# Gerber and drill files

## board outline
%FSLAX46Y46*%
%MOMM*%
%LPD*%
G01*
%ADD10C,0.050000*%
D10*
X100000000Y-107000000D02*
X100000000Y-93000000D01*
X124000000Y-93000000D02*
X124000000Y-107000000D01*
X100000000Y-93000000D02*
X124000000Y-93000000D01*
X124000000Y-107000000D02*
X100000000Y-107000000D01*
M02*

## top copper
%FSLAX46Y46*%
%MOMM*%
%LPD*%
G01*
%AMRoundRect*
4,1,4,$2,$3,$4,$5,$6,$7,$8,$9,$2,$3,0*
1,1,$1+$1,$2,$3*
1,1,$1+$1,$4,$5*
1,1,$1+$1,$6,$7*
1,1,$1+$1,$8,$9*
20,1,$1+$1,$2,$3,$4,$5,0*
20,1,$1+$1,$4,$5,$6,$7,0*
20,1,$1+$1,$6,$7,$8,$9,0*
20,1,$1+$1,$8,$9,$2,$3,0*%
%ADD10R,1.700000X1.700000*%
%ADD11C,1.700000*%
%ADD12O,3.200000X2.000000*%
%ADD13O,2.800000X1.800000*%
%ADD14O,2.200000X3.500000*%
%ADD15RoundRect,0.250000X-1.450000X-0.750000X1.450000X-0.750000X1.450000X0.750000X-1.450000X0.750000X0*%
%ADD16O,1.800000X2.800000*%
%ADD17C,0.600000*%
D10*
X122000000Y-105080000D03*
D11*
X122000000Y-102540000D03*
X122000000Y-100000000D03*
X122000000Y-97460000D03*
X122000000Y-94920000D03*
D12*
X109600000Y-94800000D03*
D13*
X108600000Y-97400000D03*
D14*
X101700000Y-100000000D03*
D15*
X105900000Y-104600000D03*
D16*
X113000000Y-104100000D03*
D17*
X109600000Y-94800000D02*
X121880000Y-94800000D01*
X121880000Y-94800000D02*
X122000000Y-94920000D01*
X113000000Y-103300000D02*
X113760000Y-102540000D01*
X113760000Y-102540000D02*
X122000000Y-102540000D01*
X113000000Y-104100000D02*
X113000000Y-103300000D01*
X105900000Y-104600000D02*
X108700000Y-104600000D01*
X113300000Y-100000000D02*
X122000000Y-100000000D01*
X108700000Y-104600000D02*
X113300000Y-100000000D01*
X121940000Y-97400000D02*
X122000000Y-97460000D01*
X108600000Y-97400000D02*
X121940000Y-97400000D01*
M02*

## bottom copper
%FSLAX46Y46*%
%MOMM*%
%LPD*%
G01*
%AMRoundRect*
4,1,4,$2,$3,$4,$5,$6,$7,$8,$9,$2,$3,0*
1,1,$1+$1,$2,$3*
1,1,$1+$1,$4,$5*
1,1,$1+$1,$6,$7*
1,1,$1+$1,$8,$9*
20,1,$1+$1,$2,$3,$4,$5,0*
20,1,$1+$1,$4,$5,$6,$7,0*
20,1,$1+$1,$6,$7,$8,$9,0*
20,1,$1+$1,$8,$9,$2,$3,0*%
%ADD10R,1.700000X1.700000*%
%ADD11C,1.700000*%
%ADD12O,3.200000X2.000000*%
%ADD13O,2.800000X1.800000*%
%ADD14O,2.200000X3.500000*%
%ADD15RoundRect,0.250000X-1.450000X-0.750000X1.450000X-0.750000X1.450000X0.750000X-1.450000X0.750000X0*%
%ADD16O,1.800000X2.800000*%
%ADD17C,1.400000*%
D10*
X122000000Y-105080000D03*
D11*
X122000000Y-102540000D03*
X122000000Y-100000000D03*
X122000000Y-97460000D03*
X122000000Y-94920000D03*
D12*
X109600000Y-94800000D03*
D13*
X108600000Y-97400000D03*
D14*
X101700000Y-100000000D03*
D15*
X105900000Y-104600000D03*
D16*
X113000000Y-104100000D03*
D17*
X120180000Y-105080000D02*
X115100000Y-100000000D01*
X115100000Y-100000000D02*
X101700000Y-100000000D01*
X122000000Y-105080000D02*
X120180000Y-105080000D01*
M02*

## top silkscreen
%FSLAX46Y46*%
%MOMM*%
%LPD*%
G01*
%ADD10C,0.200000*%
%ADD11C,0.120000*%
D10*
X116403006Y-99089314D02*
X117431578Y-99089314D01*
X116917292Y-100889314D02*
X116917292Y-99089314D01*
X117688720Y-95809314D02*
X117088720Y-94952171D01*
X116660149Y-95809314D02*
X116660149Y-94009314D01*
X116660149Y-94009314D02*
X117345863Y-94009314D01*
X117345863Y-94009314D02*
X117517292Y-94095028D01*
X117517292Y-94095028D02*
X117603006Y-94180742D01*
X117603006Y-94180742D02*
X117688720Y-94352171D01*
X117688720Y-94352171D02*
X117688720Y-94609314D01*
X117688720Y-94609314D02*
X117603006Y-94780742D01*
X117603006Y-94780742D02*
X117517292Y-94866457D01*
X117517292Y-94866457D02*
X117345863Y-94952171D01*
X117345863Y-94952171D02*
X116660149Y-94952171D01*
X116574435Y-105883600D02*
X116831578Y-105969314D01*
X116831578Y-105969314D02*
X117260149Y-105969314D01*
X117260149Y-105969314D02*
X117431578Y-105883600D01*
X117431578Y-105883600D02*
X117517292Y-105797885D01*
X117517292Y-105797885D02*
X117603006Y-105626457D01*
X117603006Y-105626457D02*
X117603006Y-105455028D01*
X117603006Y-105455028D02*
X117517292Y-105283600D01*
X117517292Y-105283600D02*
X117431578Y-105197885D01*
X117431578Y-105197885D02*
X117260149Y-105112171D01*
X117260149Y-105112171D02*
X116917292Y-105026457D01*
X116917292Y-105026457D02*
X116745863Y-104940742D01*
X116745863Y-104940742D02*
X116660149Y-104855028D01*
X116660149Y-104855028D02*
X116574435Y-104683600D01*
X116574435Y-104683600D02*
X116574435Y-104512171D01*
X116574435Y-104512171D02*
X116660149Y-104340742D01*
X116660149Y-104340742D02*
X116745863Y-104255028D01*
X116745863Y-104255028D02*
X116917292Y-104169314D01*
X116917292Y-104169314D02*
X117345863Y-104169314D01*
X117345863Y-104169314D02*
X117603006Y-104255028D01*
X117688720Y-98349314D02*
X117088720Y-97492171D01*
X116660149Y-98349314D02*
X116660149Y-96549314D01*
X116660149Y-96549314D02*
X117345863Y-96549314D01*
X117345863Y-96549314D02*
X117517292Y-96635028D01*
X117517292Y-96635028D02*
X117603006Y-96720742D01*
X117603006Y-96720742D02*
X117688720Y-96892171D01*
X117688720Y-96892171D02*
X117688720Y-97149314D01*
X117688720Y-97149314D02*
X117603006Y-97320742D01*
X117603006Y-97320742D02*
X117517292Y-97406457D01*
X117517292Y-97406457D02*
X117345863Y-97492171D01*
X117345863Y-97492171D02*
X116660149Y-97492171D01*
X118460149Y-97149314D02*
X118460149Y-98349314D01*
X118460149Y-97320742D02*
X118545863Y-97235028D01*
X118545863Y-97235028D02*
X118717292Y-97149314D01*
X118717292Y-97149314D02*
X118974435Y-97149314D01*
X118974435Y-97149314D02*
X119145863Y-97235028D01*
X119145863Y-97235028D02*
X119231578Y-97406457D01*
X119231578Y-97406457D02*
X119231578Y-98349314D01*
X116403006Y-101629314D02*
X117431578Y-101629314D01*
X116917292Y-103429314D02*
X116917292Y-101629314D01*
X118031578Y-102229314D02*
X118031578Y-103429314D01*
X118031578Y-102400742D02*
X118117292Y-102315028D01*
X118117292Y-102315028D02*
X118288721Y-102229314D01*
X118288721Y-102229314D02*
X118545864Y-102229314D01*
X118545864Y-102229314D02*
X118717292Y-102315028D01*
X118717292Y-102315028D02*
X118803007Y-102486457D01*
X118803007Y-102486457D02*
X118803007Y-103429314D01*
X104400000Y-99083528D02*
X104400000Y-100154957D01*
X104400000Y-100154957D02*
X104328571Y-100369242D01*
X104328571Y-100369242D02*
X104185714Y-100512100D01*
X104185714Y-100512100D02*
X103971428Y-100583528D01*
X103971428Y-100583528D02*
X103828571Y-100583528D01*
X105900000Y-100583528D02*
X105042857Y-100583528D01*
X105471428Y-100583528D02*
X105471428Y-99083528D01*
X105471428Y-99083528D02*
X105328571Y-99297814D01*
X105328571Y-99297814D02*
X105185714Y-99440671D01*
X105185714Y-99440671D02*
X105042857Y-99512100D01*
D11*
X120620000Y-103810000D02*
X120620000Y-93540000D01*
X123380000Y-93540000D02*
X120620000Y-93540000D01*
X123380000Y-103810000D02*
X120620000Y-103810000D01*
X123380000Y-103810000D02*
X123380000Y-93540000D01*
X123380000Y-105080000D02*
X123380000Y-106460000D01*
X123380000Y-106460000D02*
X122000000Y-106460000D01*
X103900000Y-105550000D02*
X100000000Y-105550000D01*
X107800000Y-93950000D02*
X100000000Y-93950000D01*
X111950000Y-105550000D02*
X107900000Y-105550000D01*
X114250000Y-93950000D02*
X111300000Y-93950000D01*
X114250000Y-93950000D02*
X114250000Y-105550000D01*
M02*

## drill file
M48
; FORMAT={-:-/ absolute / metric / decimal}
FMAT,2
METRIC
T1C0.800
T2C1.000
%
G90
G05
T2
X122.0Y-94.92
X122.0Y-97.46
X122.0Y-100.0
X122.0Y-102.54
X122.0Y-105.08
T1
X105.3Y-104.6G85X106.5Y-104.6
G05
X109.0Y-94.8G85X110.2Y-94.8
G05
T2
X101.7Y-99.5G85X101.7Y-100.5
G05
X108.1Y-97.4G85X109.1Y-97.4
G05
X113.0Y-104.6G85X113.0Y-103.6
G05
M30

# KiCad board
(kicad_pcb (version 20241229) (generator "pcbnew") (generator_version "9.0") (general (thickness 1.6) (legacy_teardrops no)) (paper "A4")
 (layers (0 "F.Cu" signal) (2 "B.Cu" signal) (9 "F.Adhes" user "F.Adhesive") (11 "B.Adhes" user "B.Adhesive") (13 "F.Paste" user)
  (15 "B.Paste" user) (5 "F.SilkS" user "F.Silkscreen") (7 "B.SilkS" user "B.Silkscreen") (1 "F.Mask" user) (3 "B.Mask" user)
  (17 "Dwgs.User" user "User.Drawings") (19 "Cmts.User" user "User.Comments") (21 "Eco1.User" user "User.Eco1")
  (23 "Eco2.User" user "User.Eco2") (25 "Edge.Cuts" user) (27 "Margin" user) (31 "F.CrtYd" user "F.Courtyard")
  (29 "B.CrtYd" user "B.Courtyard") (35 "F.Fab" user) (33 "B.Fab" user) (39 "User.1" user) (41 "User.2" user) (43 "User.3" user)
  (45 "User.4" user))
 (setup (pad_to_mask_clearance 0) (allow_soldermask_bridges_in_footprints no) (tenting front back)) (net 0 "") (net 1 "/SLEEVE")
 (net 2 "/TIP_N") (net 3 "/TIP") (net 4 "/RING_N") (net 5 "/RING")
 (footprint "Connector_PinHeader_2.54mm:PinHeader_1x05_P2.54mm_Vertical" (layer "F.Cu") (at 122 105.08 180)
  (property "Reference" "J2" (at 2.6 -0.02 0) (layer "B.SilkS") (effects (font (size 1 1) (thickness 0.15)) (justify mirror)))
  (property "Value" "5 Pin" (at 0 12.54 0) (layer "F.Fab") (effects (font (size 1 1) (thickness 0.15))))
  (fp_line (start 1.38 1.27) (end 1.38 11.54) (stroke (width 0.12) (type solid)) (layer "F.SilkS"))
  (fp_line (start -1.38 11.54) (end 1.38 11.54) (stroke (width 0.12) (type solid)) (layer "F.SilkS"))
  (fp_line (start -1.38 1.27) (end 1.38 1.27) (stroke (width 0.12) (type solid)) (layer "F.SilkS"))
  (fp_line (start -1.38 1.27) (end -1.38 11.54) (stroke (width 0.12) (type solid)) (layer "F.SilkS"))
  (fp_line (start -1.38 0) (end -1.38 -1.38) (stroke (width 0.12) (type solid)) (layer "F.SilkS"))
  (fp_line (start -1.38 -1.38) (end 0 -1.38) (stroke (width 0.12) (type solid)) (layer "F.SilkS"))
  (pad "1" thru_hole rect (at 0 0 180) (size 1.7 1.7) (drill 1) (layers "*.Cu" "*.Mask") (remove_unused_layers no) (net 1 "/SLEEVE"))
  (pad "2" thru_hole circle (at 0 2.54 180) (size 1.7 1.7) (drill 1) (layers "*.Cu" "*.Mask") (remove_unused_layers no) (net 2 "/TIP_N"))
  (pad "3" thru_hole circle (at 0 5.08 180) (size 1.7 1.7) (drill 1) (layers "*.Cu" "*.Mask") (remove_unused_layers no) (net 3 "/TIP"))
  (pad "4" thru_hole circle (at 0 7.62 180) (size 1.7 1.7) (drill 1) (layers "*.Cu" "*.Mask") (remove_unused_layers no) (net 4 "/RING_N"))
  (pad "5" thru_hole circle (at 0 10.16 180) (size 1.7 1.7) (drill 1) (layers "*.Cu" "*.Mask") (remove_unused_layers no) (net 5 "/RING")))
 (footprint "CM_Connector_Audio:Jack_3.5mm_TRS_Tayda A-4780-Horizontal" (layer "F.Cu") (at 101.7 100)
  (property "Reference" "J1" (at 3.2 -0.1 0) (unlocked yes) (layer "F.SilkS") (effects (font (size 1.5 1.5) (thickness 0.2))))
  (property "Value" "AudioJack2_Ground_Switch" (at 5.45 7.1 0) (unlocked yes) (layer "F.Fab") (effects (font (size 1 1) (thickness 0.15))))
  (fp_line (start 2.2 5.55) (end -1.7 5.55) (stroke (width 0.12) (type solid)) (layer "F.SilkS"))
  (fp_line (start 6.1 -6.05) (end -1.7 -6.05) (stroke (width 0.12) (type solid)) (layer "F.SilkS"))
  (fp_line (start 10.25 5.55) (end 6.2 5.55) (stroke (width 0.12) (type solid)) (layer "F.SilkS"))
  (fp_line (start 12.55 -6.05) (end 9.6 -6.05) (stroke (width 0.12) (type solid)) (layer "F.SilkS"))
  (fp_line (start 12.55 -6.05) (end 12.55 5.55) (stroke (width 0.12) (type solid)) (layer "F.SilkS"))
  (pad "R" thru_hole oval (at 7.9 -5.2) (size 3.2 2) (drill oval 2 0.8) (layers "*.Cu" "*.Mask") (remove_unused_layers no) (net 5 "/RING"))
  (pad "RN" thru_hole oval (at 6.9 -2.6) (size 2.8 1.8) (drill oval 2 1) (layers "*.Cu" "*.Mask") (remove_unused_layers no)
   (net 4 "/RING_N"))
  (pad "S" thru_hole oval (at 0 0 270) (size 3.5 2.2) (drill oval 2 1) (layers "*.Cu" "*.Mask") (remove_unused_layers no) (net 1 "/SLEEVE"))
  (pad "T" thru_hole roundrect (at 4.2 4.6) (size 3.4 2) (drill oval 2 0.8) (layers "*.Cu" "*.Mask") (remove_unused_layers no)
   (roundrect_rratio 0.125) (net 3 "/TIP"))
  (pad "TN" thru_hole oval (at 11.3 4.1 90) (size 2.8 1.8) (drill oval 2 1) (layers "*.Cu" "*.Mask") (remove_unused_layers no)
   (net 2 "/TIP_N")))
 (gr_line (start 100 107) (end 100 93) (stroke (width 0.05) (type default)) (layer "Edge.Cuts"))
 (gr_line (start 124 93) (end 124 107) (stroke (width 0.05) (type default)) (layer "Edge.Cuts"))
 (gr_line (start 100 93) (end 124 93) (stroke (width 0.05) (type default)) (layer "Edge.Cuts"))
 (gr_line (start 124 107) (end 100 107) (stroke (width 0.05) (type default)) (layer "Edge.Cuts"))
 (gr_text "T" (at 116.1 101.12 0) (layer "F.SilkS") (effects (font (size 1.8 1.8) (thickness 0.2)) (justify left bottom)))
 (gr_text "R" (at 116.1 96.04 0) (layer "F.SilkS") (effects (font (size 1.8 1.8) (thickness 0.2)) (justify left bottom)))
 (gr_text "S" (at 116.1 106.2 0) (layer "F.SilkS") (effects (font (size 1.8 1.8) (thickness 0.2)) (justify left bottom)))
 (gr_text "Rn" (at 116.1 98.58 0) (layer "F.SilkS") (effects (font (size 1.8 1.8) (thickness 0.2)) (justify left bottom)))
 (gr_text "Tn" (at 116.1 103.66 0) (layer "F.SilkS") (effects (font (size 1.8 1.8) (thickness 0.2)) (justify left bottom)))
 (segment (start 109.6 94.8) (end 121.88 94.8) (width 0.6) (layer "F.Cu") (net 5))
 (segment (start 121.88 94.8) (end 122 94.92) (width 0.6) (layer "F.Cu") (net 5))
 (segment (start 113 103.3) (end 113.76 102.54) (width 0.6) (layer "F.Cu") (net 2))
 (segment (start 113.76 102.54) (end 122 102.54) (width 0.6) (layer "F.Cu") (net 2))
 (segment (start 113 104.1) (end 113 103.3) (width 0.6) (layer "F.Cu") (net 2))
 (segment (start 105.9 104.6) (end 108.7 104.6) (width 0.6) (layer "F.Cu") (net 3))
 (segment (start 113.3 100) (end 122 100) (width 0.6) (layer "F.Cu") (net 3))
 (segment (start 108.7 104.6) (end 113.3 100) (width 0.6) (layer "F.Cu") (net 3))
 (segment (start 120.18 105.08) (end 115.1 100) (width 1.4) (layer "B.Cu") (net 1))
 (segment (start 115.1 100) (end 101.7 100) (width 1.4) (layer "B.Cu") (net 1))
 (segment (start 122 105.08) (end 120.18 105.08) (width 1.4) (layer "B.Cu") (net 1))
 (segment (start 121.94 97.4) (end 122 97.46) (width 0.6) (layer "F.Cu") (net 4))
 (segment (start 108.6 97.4) (end 121.94 97.4) (width 0.6) (layer "F.Cu") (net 4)))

